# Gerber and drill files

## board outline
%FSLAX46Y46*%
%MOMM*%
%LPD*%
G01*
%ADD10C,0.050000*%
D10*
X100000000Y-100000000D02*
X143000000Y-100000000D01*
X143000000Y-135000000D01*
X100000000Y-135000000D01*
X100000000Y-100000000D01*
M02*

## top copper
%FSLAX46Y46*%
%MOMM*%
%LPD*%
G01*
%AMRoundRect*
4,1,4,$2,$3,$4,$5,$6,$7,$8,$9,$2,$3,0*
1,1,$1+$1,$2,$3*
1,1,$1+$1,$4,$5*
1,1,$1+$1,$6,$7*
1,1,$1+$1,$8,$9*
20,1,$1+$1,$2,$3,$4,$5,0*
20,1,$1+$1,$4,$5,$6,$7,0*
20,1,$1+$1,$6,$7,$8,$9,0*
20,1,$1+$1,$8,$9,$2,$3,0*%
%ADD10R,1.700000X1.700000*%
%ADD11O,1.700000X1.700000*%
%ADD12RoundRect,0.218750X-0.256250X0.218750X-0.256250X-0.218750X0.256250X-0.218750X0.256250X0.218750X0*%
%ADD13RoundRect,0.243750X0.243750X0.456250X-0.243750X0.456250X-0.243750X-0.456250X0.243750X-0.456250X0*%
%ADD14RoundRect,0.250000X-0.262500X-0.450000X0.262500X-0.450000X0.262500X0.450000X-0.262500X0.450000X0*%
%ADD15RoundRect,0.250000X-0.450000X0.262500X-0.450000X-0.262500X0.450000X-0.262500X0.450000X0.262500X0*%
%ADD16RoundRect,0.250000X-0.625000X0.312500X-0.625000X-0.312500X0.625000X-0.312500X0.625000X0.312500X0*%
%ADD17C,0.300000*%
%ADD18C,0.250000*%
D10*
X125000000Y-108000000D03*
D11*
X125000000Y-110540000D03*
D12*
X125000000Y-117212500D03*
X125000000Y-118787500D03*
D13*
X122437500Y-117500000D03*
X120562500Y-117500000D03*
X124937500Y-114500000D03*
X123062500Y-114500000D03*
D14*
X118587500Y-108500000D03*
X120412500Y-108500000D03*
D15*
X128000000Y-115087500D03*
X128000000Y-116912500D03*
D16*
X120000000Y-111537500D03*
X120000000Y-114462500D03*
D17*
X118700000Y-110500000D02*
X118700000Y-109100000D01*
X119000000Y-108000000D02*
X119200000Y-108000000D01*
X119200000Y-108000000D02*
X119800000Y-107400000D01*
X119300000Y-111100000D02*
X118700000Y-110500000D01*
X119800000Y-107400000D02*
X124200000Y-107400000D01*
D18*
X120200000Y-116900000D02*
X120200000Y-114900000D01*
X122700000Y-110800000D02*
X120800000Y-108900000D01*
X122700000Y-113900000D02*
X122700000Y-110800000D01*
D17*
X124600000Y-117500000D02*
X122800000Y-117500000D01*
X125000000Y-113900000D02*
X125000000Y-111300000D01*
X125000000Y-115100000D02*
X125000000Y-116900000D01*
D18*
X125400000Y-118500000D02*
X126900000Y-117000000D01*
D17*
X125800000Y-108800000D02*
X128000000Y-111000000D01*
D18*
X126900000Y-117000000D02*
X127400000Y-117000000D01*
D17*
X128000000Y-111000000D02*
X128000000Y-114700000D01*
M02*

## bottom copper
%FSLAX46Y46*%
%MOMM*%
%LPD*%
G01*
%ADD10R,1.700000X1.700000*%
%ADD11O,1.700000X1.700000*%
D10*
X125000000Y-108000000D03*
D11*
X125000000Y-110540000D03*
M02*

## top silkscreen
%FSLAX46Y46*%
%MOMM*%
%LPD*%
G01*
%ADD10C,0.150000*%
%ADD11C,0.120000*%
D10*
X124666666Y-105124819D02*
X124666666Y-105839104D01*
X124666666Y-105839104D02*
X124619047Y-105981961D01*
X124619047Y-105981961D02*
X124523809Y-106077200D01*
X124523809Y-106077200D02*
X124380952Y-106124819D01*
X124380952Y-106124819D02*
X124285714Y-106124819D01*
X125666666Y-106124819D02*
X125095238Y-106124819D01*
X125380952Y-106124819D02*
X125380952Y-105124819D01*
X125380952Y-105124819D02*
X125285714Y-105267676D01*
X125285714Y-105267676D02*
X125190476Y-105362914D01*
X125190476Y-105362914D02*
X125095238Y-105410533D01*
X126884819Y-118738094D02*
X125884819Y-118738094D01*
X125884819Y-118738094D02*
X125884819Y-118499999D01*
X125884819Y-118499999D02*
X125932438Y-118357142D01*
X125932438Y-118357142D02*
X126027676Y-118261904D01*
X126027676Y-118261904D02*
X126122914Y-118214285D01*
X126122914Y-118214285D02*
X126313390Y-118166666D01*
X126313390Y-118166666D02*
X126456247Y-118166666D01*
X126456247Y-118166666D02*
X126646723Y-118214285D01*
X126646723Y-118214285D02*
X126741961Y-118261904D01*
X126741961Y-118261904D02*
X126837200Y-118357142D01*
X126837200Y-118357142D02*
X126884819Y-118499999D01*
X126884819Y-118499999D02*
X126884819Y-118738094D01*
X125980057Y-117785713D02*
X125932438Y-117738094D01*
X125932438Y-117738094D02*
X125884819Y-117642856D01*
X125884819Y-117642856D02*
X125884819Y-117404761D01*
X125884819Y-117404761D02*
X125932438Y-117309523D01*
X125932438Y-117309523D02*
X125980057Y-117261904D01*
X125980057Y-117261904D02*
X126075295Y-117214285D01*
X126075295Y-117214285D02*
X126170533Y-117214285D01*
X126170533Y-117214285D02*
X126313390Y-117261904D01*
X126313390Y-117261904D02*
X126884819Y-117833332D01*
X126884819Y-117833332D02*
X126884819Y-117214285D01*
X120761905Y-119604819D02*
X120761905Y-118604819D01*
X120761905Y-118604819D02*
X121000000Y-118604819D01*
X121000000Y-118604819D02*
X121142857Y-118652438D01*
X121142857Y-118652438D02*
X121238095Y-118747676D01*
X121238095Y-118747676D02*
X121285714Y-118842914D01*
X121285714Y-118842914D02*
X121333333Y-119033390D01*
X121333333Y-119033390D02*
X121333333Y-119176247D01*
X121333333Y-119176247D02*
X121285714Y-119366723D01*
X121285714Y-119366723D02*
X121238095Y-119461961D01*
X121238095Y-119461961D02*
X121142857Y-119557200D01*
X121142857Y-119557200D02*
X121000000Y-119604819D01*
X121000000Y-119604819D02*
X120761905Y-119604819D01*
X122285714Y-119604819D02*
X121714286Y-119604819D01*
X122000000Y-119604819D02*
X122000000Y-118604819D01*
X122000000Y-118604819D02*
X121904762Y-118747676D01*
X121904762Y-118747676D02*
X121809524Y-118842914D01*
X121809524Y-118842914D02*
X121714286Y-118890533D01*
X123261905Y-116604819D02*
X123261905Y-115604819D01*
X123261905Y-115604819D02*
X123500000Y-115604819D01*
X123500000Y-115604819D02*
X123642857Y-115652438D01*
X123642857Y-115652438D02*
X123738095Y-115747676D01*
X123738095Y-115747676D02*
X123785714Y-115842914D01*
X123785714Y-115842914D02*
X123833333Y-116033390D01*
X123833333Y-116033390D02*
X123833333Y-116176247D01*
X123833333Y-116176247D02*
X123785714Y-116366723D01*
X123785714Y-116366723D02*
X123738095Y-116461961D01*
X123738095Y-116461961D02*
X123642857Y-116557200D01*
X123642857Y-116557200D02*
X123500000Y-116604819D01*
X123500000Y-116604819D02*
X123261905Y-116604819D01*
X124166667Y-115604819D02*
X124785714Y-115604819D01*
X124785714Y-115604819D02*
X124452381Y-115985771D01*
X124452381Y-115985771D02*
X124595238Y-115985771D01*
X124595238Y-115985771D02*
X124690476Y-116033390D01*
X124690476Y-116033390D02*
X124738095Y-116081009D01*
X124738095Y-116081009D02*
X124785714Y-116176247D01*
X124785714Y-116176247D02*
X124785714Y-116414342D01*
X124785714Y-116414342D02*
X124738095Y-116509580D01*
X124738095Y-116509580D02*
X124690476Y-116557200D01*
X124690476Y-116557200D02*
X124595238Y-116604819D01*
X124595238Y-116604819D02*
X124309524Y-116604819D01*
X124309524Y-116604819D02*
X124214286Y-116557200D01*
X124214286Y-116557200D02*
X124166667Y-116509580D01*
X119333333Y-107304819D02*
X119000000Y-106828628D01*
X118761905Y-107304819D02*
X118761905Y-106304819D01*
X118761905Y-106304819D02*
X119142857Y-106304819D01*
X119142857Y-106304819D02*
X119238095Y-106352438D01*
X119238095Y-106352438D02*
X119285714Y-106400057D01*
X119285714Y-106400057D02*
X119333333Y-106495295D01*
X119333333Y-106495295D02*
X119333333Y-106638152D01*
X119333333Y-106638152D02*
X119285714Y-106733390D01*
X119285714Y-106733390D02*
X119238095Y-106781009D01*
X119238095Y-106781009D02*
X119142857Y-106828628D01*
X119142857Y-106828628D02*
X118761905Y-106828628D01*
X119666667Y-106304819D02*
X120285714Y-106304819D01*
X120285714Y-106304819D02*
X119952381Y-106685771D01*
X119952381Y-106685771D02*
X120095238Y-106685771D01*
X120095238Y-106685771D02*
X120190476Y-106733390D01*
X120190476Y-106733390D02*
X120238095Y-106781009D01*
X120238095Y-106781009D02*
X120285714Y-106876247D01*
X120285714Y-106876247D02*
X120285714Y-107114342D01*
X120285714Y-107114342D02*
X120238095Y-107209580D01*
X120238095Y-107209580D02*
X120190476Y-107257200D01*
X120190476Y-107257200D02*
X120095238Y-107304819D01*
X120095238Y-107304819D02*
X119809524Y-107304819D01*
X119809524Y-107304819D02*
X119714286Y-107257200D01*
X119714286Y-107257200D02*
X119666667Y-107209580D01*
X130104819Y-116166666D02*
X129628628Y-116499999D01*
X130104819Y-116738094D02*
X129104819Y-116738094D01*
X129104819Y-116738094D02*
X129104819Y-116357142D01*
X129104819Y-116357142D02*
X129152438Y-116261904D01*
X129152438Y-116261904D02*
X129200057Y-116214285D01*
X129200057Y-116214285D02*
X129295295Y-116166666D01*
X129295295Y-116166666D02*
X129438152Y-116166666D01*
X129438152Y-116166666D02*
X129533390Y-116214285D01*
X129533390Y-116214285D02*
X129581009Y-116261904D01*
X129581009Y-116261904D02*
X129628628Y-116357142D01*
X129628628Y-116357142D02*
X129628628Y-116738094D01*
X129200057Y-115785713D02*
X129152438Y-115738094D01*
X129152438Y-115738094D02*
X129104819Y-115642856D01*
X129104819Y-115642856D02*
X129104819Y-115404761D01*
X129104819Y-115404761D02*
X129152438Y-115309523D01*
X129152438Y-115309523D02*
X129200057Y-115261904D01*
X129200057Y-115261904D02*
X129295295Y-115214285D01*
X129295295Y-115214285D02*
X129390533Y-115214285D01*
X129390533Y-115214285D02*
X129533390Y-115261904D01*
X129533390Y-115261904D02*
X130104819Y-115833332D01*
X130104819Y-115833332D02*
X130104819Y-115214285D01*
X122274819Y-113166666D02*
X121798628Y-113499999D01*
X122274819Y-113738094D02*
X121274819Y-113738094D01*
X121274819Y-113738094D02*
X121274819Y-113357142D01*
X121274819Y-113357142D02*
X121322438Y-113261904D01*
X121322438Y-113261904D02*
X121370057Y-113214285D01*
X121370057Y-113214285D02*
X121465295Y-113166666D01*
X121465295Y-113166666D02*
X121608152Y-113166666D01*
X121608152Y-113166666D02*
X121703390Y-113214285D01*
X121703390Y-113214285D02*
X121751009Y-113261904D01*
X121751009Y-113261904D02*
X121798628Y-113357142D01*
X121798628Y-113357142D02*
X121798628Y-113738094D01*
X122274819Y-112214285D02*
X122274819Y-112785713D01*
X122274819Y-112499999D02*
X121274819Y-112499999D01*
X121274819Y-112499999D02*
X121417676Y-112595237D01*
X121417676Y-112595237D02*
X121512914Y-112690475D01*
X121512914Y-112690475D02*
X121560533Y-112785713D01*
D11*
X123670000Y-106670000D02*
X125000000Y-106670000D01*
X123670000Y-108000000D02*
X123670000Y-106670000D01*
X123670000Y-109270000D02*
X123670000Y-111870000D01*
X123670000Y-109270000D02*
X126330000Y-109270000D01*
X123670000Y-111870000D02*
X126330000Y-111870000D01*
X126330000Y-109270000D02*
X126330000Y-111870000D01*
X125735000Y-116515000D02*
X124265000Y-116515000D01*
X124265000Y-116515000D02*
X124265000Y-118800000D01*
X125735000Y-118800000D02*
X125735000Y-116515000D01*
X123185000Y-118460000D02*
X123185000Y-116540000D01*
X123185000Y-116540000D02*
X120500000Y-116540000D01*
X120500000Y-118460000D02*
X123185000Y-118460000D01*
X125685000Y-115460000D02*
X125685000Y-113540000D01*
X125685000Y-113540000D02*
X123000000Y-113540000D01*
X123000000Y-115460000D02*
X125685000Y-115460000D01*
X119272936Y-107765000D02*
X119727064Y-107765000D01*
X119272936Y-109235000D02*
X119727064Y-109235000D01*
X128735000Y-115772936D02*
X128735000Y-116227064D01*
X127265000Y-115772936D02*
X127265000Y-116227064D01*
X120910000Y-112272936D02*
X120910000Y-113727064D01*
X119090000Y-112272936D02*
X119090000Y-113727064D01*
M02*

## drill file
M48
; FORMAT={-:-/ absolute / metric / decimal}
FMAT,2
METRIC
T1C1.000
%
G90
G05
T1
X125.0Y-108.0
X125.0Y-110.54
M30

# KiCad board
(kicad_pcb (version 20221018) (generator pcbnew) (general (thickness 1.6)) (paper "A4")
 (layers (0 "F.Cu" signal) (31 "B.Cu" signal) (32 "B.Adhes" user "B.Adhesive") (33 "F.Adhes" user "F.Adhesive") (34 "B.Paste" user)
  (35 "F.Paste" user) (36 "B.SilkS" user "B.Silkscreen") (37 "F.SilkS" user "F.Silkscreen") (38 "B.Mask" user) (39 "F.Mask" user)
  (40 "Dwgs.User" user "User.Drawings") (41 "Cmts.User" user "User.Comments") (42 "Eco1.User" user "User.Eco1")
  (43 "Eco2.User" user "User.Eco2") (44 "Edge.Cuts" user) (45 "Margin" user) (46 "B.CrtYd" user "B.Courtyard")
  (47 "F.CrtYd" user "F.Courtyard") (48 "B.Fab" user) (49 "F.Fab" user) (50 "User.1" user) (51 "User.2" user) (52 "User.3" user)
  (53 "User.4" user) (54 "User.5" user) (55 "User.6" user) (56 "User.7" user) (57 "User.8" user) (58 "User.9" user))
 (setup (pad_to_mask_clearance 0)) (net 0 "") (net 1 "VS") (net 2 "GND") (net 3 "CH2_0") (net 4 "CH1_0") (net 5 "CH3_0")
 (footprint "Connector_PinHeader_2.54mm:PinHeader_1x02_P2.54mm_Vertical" (layer "F.Cu") (at 125 108)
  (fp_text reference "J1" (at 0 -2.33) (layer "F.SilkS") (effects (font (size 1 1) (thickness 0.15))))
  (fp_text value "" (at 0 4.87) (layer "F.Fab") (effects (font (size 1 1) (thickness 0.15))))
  (fp_line (start -1.33 -1.33) (end 0 -1.33) (stroke (width 0.12) (type solid)) (layer "F.SilkS"))
  (fp_line (start -1.33 0) (end -1.33 -1.33) (stroke (width 0.12) (type solid)) (layer "F.SilkS"))
  (fp_line (start -1.33 1.27) (end -1.33 3.87) (stroke (width 0.12) (type solid)) (layer "F.SilkS"))
  (fp_line (start -1.33 1.27) (end 1.33 1.27) (stroke (width 0.12) (type solid)) (layer "F.SilkS"))
  (fp_line (start -1.33 3.87) (end 1.33 3.87) (stroke (width 0.12) (type solid)) (layer "F.SilkS"))
  (fp_line (start 1.33 1.27) (end 1.33 3.87) (stroke (width 0.12) (type solid)) (layer "F.SilkS"))
  (pad "1" thru_hole rect (at 0 0) (size 1.7 1.7) (drill 1) (layers "*.Cu" "*.Mask") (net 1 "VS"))
  (pad "2" thru_hole oval (at 0 2.54) (size 1.7 1.7) (drill 1) (layers "*.Cu" "*.Mask") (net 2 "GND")))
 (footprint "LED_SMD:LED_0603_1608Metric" (layer "F.Cu") (at 125 118 -90)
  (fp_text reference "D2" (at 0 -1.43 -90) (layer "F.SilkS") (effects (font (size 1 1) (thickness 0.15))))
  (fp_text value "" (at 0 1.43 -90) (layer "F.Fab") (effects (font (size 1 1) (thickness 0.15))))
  (fp_line (start -1.485 -0.735) (end -1.485 0.735) (stroke (width 0.12) (type solid)) (layer "F.SilkS"))
  (fp_line (start -1.485 0.735) (end 0.8 0.735) (stroke (width 0.12) (type solid)) (layer "F.SilkS"))
  (fp_line (start 0.8 -0.735) (end -1.485 -0.735) (stroke (width 0.12) (type solid)) (layer "F.SilkS"))
  (pad "1" smd roundrect (at -0.7875 0 270) (size 0.875 0.95) (layers "F.Cu" "F.Paste" "F.Mask") (roundrect_rratio 0.25) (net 2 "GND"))
  (pad "2" smd roundrect (at 0.7875 0 270) (size 0.875 0.95) (layers "F.Cu" "F.Paste" "F.Mask") (roundrect_rratio 0.25) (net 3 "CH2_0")))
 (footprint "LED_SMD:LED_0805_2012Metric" (layer "F.Cu") (at 121.5 117.5 180)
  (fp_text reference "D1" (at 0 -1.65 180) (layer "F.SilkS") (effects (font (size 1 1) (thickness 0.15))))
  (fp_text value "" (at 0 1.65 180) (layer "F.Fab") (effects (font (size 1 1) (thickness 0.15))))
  (fp_line (start -1.685 -0.96) (end -1.685 0.96) (stroke (width 0.12) (type solid)) (layer "F.SilkS"))
  (fp_line (start -1.685 0.96) (end 1 0.96) (stroke (width 0.12) (type solid)) (layer "F.SilkS"))
  (fp_line (start 1 -0.96) (end -1.685 -0.96) (stroke (width 0.12) (type solid)) (layer "F.SilkS"))
  (pad "1" smd roundrect (at -0.9375 0 180) (size 0.975 1.4) (layers "F.Cu" "F.Paste" "F.Mask") (roundrect_rratio 0.25) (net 2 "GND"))
  (pad "2" smd roundrect (at 0.9375 0 180) (size 0.975 1.4) (layers "F.Cu" "F.Paste" "F.Mask") (roundrect_rratio 0.25) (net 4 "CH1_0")))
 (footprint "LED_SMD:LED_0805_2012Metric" (layer "F.Cu") (at 124 114.5 180)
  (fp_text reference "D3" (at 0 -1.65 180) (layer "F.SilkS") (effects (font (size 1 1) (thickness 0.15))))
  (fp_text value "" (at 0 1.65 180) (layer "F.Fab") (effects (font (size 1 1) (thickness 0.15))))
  (fp_line (start -1.685 -0.96) (end -1.685 0.96) (stroke (width 0.12) (type solid)) (layer "F.SilkS"))
  (fp_line (start -1.685 0.96) (end 1 0.96) (stroke (width 0.12) (type solid)) (layer "F.SilkS"))
  (fp_line (start 1 -0.96) (end -1.685 -0.96) (stroke (width 0.12) (type solid)) (layer "F.SilkS"))
  (pad "1" smd roundrect (at -0.9375 0 180) (size 0.975 1.4) (layers "F.Cu" "F.Paste" "F.Mask") (roundrect_rratio 0.25) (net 2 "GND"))
  (pad "2" smd roundrect (at 0.9375 0 180) (size 0.975 1.4) (layers "F.Cu" "F.Paste" "F.Mask") (roundrect_rratio 0.25) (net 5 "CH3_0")))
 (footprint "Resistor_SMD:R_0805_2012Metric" (layer "F.Cu") (at 119.5 108.5)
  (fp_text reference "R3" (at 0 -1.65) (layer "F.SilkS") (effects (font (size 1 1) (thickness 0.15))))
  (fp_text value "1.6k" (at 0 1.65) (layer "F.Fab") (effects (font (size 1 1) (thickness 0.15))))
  (fp_line (start -0.227064 -0.735) (end 0.227064 -0.735) (stroke (width 0.12) (type solid)) (layer "F.SilkS"))
  (fp_line (start -0.227064 0.735) (end 0.227064 0.735) (stroke (width 0.12) (type solid)) (layer "F.SilkS"))
  (pad "1" smd roundrect (at -0.9125 0) (size 1.025 1.4) (layers "F.Cu" "F.Paste" "F.Mask") (roundrect_rratio 0.243902) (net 1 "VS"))
  (pad "2" smd roundrect (at 0.9125 0) (size 1.025 1.4) (layers "F.Cu" "F.Paste" "F.Mask") (roundrect_rratio 0.243902) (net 5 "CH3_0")))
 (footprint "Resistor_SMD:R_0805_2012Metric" (layer "F.Cu") (at 128 116 -90)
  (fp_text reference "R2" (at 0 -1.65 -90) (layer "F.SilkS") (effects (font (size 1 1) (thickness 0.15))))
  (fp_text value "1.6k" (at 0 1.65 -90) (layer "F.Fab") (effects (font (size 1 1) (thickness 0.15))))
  (fp_line (start -0.227064 -0.735) (end 0.227064 -0.735) (stroke (width 0.12) (type solid)) (layer "F.SilkS"))
  (fp_line (start -0.227064 0.735) (end 0.227064 0.735) (stroke (width 0.12) (type solid)) (layer "F.SilkS"))
  (pad "1" smd roundrect (at -0.9125 0 270) (size 1.025 1.4) (layers "F.Cu" "F.Paste" "F.Mask") (roundrect_rratio 0.243902) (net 1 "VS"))
  (pad "2" smd roundrect (at 0.9125 0 270) (size 1.025 1.4) (layers "F.Cu" "F.Paste" "F.Mask") (roundrect_rratio 0.243902) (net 3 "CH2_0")))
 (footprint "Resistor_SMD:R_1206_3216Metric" (layer "F.Cu") (at 120 113 -90)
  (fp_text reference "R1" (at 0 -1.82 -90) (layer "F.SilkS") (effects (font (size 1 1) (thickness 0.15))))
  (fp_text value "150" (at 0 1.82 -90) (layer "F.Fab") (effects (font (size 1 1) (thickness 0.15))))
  (fp_line (start -0.727064 -0.91) (end 0.727064 -0.91) (stroke (width 0.12) (type solid)) (layer "F.SilkS"))
  (fp_line (start -0.727064 0.91) (end 0.727064 0.91) (stroke (width 0.12) (type solid)) (layer "F.SilkS"))
  (pad "1" smd roundrect (at -1.4625 0 270) (size 1.125 1.75) (layers "F.Cu" "F.Paste" "F.Mask") (roundrect_rratio 0.222222) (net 1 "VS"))
  (pad "2" smd roundrect (at 1.4625 0 270) (size 1.125 1.75) (layers "F.Cu" "F.Paste" "F.Mask") (roundrect_rratio 0.222222) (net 4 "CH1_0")))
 (gr_rect (start 100 100) (end 143 135) (stroke (width 0.05) (type default)) (fill none) (layer "Edge.Cuts"))
 (segment (start 118.7 110.5) (end 118.7 109.1) (width 0.3) (layer "F.Cu") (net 1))
 (segment (start 119 108) (end 119.2 108) (width 0.3) (layer "F.Cu") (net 1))
 (segment (start 119.2 108) (end 119.8 107.4) (width 0.3) (layer "F.Cu") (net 1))
 (segment (start 119.3 111.1) (end 118.7 110.5) (width 0.3) (layer "F.Cu") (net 1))
 (segment (start 119.8 107.4) (end 124.2 107.4) (width 0.3) (layer "F.Cu") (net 1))
 (segment (start 120.2 116.9) (end 120.2 114.9) (width 0.25) (layer "F.Cu") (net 4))
 (segment (start 122.7 110.8) (end 120.8 108.9) (width 0.25) (layer "F.Cu") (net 5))
 (segment (start 122.7 113.9) (end 122.7 110.8) (width 0.25) (layer "F.Cu") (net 5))
 (segment (start 124.6 117.5) (end 122.8 117.5) (width 0.3) (layer "F.Cu") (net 2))
 (segment (start 125 113.9) (end 125 111.3) (width 0.3) (layer "F.Cu") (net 2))
 (segment (start 125 115.1) (end 125 116.9) (width 0.3) (layer "F.Cu") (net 2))
 (segment (start 125.4 118.5) (end 126.9 117) (width 0.25) (layer "F.Cu") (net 3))
 (segment (start 125.8 108.8) (end 128 111) (width 0.3) (layer "F.Cu") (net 1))
 (segment (start 126.9 117) (end 127.4 117) (width 0.25) (layer "F.Cu") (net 3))
 (segment (start 128 111) (end 128 114.7) (width 0.3) (layer "F.Cu") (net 1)))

